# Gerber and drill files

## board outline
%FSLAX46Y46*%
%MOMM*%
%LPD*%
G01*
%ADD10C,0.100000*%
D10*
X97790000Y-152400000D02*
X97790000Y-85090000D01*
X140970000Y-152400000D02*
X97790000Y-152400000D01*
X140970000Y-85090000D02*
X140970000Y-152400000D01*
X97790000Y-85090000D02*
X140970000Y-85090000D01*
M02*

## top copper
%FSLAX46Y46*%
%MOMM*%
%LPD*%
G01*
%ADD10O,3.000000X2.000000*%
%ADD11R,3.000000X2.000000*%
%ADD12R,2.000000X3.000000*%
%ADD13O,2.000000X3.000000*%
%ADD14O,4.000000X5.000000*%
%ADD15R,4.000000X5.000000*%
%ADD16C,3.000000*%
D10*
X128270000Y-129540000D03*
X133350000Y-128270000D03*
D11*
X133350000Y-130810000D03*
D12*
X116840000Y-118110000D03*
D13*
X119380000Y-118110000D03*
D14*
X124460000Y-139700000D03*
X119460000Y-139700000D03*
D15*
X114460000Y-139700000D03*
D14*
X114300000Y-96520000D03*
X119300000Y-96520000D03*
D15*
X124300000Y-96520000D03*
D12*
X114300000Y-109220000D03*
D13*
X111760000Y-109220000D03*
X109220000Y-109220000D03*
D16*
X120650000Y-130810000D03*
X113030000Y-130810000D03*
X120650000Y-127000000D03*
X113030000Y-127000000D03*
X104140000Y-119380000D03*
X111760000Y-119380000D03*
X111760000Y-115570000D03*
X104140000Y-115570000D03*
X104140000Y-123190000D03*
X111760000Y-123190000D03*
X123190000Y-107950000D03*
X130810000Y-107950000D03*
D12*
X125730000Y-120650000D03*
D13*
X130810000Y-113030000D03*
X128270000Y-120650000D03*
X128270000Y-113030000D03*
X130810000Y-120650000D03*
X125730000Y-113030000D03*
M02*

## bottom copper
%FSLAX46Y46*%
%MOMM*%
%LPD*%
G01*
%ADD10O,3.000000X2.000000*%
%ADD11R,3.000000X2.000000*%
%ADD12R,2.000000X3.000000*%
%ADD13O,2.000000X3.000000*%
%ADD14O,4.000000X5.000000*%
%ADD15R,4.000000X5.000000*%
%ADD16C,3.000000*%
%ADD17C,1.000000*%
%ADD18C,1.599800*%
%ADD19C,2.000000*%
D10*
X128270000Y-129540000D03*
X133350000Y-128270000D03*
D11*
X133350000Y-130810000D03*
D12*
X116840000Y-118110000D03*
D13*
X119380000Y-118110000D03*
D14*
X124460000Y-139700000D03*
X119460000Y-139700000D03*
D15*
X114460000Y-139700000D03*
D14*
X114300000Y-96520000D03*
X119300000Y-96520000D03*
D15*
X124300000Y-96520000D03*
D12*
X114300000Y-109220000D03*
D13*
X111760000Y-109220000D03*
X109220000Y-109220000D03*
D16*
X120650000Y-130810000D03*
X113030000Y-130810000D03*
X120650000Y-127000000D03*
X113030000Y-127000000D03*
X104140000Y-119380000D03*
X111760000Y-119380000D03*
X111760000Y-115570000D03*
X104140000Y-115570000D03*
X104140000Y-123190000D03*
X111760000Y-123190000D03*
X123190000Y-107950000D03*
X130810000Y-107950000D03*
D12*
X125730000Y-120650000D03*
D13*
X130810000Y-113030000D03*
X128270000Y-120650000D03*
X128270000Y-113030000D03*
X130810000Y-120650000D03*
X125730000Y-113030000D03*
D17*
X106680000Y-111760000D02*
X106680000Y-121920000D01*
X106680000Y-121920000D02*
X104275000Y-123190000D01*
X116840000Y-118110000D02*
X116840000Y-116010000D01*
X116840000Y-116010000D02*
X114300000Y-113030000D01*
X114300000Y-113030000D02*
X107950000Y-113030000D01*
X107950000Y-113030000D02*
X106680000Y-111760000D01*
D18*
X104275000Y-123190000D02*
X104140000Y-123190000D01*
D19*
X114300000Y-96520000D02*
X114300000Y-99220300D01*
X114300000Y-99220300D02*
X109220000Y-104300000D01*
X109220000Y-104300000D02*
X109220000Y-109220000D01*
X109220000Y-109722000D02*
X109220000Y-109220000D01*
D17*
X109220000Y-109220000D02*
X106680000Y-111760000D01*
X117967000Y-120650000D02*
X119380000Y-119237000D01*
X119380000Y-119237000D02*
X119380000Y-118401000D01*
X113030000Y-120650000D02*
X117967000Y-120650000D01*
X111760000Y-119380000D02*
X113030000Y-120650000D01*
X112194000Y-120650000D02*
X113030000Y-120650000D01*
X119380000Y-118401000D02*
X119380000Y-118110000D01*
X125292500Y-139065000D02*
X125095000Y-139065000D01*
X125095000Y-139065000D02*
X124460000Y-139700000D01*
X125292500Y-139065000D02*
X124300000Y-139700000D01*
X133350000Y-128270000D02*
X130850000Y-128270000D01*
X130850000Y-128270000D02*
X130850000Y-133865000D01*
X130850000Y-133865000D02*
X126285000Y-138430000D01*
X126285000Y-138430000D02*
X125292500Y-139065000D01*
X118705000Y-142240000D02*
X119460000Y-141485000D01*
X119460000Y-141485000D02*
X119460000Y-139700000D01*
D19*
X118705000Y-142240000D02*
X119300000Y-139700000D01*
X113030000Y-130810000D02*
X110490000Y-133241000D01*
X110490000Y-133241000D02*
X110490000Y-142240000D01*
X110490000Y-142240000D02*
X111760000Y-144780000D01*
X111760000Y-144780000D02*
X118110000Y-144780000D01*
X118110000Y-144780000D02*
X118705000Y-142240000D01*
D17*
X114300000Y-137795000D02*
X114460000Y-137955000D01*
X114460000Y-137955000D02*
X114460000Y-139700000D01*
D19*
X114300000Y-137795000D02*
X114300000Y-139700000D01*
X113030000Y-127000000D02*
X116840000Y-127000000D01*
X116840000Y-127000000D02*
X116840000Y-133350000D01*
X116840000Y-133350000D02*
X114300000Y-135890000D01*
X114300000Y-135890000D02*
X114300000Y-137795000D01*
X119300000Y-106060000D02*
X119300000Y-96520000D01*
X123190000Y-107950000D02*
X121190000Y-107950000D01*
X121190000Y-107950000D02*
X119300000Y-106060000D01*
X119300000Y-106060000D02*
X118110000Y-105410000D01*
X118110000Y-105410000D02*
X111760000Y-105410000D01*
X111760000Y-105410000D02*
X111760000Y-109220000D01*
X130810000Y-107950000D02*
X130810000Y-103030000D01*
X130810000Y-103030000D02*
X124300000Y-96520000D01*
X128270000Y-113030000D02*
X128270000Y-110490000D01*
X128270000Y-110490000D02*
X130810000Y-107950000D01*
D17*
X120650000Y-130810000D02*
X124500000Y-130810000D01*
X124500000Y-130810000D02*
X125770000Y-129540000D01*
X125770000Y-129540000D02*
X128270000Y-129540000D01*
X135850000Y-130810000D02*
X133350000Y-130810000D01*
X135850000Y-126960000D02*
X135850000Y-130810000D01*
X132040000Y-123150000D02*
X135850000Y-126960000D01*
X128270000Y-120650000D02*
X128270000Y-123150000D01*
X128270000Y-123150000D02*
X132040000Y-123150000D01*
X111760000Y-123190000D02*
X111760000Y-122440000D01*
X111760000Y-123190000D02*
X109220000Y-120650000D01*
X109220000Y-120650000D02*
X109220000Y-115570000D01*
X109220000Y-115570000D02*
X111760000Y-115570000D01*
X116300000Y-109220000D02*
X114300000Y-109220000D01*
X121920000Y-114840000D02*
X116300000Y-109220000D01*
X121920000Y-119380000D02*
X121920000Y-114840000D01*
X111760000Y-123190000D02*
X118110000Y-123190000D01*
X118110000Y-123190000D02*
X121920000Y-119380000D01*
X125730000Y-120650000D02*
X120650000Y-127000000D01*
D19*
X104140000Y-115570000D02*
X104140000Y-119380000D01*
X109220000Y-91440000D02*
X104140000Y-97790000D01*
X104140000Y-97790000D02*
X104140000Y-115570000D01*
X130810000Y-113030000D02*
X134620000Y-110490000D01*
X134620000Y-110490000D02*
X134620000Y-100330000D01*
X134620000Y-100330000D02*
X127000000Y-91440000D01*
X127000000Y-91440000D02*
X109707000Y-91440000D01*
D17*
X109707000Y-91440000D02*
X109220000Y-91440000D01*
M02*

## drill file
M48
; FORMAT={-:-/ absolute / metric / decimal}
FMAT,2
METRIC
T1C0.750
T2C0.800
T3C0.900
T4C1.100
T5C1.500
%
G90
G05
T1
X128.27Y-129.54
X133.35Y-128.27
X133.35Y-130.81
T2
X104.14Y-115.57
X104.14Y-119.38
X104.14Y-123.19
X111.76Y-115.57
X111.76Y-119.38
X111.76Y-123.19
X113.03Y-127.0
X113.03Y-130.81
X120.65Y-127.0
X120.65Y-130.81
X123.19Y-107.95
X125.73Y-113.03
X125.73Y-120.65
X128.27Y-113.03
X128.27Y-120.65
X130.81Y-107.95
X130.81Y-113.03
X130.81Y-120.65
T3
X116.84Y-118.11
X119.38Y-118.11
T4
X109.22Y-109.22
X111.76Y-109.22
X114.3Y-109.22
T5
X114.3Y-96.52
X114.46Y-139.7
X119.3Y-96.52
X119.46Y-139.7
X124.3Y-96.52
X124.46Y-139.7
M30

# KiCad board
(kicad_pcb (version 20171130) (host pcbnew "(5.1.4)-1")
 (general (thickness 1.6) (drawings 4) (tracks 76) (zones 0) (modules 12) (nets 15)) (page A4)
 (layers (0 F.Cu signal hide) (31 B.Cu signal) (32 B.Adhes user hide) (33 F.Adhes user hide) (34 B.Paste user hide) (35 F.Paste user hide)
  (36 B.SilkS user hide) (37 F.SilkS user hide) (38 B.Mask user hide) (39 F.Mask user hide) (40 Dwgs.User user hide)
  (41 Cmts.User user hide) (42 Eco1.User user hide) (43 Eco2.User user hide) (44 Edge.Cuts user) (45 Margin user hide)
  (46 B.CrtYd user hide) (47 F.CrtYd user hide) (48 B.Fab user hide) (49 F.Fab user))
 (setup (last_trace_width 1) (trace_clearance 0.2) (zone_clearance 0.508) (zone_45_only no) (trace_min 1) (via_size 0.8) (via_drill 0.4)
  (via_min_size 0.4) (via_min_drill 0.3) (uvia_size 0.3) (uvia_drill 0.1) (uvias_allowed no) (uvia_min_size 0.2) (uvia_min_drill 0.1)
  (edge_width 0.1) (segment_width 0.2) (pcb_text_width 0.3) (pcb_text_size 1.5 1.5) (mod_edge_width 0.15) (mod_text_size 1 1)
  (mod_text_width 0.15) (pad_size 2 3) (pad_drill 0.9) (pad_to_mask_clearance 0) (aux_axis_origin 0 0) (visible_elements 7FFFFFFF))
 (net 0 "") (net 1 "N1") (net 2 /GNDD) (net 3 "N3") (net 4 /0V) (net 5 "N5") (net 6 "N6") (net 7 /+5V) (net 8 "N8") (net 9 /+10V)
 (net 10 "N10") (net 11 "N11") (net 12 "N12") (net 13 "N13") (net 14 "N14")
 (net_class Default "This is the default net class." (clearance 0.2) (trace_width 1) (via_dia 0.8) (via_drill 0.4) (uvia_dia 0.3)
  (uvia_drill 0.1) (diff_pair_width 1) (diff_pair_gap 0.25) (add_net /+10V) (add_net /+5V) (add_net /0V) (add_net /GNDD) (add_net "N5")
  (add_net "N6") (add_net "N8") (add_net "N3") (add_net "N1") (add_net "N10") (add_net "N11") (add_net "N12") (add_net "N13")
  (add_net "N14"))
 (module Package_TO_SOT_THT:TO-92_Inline (layer F.Cu) (at 133.35 130.81 90)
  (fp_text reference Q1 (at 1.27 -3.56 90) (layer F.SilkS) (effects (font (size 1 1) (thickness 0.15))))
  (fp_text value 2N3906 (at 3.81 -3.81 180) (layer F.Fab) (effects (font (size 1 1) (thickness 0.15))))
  (pad 2 thru_hole oval (at 1.27 -5.08 90) (size 2 3) (drill 0.75) (layers *.Cu *.Mask) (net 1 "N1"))
  (pad 3 thru_hole oval (at 2.54 0 90) (size 2 3) (drill 0.75) (layers *.Cu *.Mask) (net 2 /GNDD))
  (pad 1 thru_hole rect (at 0 0 90) (size 2 3) (drill 0.75) (layers *.Cu *.Mask) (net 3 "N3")))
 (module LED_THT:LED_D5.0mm (layer F.Cu) (at 116.84 118.11)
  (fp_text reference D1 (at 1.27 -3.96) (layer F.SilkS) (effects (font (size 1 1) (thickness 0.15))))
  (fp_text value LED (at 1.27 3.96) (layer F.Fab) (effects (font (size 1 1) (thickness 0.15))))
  (pad 1 thru_hole rect (at 0 0) (size 2 3) (drill 0.9) (layers *.Cu *.Mask) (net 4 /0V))
  (pad 2 thru_hole oval (at 2.54 0) (size 2 3) (drill 0.9) (layers *.Cu *.Mask) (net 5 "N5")))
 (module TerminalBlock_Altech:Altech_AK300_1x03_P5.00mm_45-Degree (layer F.Cu) (at 114.46 139.7)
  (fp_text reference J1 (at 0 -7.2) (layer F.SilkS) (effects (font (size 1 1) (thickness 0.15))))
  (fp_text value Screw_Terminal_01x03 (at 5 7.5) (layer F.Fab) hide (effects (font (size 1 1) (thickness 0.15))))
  (pad 3 thru_hole oval (at 10 0) (size 4 5) (drill 1.5) (layers *.Cu *.Mask) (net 2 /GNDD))
  (pad 2 thru_hole oval (at 5 0) (size 4 5) (drill 1.5) (layers *.Cu *.Mask) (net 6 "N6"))
  (pad 1 thru_hole rect (at 0 0) (size 4 5) (drill 1.5) (layers *.Cu *.Mask) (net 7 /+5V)))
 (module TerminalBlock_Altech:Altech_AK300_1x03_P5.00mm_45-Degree (layer F.Cu) (at 114.3 96.52)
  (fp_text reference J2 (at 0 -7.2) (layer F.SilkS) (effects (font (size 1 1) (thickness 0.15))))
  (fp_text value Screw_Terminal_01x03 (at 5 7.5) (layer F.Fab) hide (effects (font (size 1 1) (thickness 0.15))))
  (pad 1 thru_hole oval (at 0 0) (size 4 5) (drill 1.5) (layers *.Cu *.Mask) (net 4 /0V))
  (pad 2 thru_hole oval (at 5 0) (size 4 5) (drill 1.5) (layers *.Cu *.Mask) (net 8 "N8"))
  (pad 3 thru_hole rect (at 10 0) (size 4 5) (drill 1.5) (layers *.Cu *.Mask) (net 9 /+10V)))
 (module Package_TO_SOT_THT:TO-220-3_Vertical (layer F.Cu) (at 114.3 109.22 180)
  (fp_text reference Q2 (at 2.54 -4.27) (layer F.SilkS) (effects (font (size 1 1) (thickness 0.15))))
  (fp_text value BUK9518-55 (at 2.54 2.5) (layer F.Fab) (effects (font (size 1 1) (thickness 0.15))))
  (pad 1 thru_hole rect (at 0 0 180) (size 2 3) (drill 1.1) (layers *.Cu *.Mask) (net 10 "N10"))
  (pad 2 thru_hole oval (at 2.54 0 180) (size 2 3) (drill 1.1) (layers *.Cu *.Mask) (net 8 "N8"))
  (pad 3 thru_hole oval (at 5.08 0 180) (size 2 3) (drill 1.1) (layers *.Cu *.Mask) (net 4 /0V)))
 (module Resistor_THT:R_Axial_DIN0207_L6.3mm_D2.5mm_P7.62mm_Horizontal (layer F.Cu) (at 120.65 130.81 180)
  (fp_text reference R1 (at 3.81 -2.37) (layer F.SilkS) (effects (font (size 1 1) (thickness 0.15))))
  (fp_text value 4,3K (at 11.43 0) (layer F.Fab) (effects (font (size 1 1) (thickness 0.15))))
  (pad 1 thru_hole circle (at 0 0 180) (size 3 3) (drill 0.8) (layers *.Cu *.Mask) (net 1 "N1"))
  (pad 2 thru_hole circle (at 7.62 0 180) (size 3 3) (drill 0.8) (layers *.Cu *.Mask) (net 6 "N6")))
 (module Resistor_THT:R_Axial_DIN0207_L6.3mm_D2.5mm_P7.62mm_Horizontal (layer F.Cu) (at 120.65 127 180)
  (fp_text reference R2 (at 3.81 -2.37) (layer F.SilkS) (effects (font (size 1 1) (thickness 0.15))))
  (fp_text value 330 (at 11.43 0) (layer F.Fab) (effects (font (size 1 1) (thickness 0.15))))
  (pad 1 thru_hole circle (at 0 0 180) (size 3 3) (drill 0.8) (layers *.Cu *.Mask) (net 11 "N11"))
  (pad 2 thru_hole circle (at 7.62 0 180) (size 3 3) (drill 0.8) (layers *.Cu *.Mask) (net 7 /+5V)))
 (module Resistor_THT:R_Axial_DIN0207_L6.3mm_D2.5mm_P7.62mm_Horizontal (layer F.Cu) (at 111.76 119.38 180)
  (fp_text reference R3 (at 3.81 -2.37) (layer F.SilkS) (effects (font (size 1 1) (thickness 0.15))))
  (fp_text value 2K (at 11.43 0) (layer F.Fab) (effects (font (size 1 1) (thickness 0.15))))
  (pad 2 thru_hole circle (at 7.62 0 180) (size 3 3) (drill 0.8) (layers *.Cu *.Mask) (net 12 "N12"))
  (pad 1 thru_hole circle (at 0 0 180) (size 3 3) (drill 0.8) (layers *.Cu *.Mask) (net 5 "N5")))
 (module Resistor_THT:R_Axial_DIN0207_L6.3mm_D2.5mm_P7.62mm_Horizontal (layer F.Cu) (at 104.14 115.57)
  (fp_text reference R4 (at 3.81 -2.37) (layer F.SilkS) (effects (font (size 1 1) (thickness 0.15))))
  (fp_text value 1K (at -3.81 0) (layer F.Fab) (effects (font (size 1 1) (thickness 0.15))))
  (pad 2 thru_hole circle (at 7.62 0) (size 3 3) (drill 0.8) (layers *.Cu *.Mask) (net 10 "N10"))
  (pad 1 thru_hole circle (at 0 0) (size 3 3) (drill 0.8) (layers *.Cu *.Mask) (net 12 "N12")))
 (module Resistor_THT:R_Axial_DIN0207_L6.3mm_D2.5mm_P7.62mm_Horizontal (layer F.Cu) (at 104.14 123.19)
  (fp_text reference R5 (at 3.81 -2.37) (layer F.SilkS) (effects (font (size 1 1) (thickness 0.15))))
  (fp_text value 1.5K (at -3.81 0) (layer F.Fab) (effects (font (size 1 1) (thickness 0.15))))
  (pad 1 thru_hole circle (at 0 0) (size 3 3) (drill 0.8) (layers *.Cu *.Mask) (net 4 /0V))
  (pad 2 thru_hole circle (at 7.62 0) (size 3 3) (drill 0.8) (layers *.Cu *.Mask) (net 10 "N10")))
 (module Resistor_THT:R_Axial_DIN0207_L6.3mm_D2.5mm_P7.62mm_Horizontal (layer F.Cu) (at 130.81 107.95 180)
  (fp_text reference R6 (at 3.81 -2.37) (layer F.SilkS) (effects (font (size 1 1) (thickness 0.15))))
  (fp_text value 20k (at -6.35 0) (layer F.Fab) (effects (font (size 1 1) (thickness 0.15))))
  (pad 2 thru_hole circle (at 7.62 0 180) (size 3 3) (drill 0.8) (layers *.Cu *.Mask) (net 8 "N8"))
  (pad 1 thru_hole circle (at 0 0 180) (size 3 3) (drill 0.8) (layers *.Cu *.Mask) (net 9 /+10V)))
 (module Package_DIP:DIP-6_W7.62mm (layer F.Cu) (at 125.73 120.65 90)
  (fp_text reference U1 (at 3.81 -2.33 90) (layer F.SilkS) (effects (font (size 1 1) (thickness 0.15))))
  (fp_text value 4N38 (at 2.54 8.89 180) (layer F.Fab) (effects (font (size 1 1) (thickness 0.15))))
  (pad 1 thru_hole rect (at 0 0 90) (size 3 2) (drill 0.8) (layers *.Cu *.Mask) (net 11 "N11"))
  (pad 4 thru_hole oval (at 7.62 5.08 90) (size 3 2) (drill 0.8) (layers *.Cu *.Mask) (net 12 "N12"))
  (pad 2 thru_hole oval (at 0 2.54 90) (size 3 2) (drill 0.8) (layers *.Cu *.Mask) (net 3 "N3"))
  (pad 5 thru_hole oval (at 7.62 2.54 90) (size 3 2) (drill 0.8) (layers *.Cu *.Mask) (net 9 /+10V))
  (pad 3 thru_hole oval (at 0 5.08 90) (size 3 2) (drill 0.8) (layers *.Cu *.Mask) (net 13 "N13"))
  (pad 6 thru_hole oval (at 7.62 0 90) (size 3 2) (drill 0.8) (layers *.Cu *.Mask) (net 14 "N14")))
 (gr_line (start 97.79 152.4) (end 97.79 85.09) (layer Edge.Cuts) (width 0.1))
 (gr_line (start 140.97 152.4) (end 97.79 152.4) (layer Edge.Cuts) (width 0.1))
 (gr_line (start 140.97 85.09) (end 140.97 152.4) (layer Edge.Cuts) (width 0.1))
 (gr_line (start 97.79 85.09) (end 140.97 85.09) (layer Edge.Cuts) (width 0.1))
 (segment (start 106.68 111.76) (end 106.68 121.92) (width 1) (layer B.Cu) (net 4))
 (segment (start 106.68 121.92) (end 104.275 123.19) (width 1) (layer B.Cu) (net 4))
 (segment (start 116.84 118.11) (end 116.84 116.01) (width 1) (layer B.Cu) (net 4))
 (segment (start 116.84 116.01) (end 114.3 113.03) (width 1) (layer B.Cu) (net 4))
 (segment (start 114.3 113.03) (end 107.95 113.03) (width 1) (layer B.Cu) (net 4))
 (segment (start 107.95 113.03) (end 106.68 111.76) (width 1) (layer B.Cu) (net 4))
 (segment (start 104.275 123.19) (end 104.14 123.19) (width 1.5998) (layer B.Cu) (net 4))
 (segment (start 114.3 96.52) (end 114.3 99.2203) (width 2) (layer B.Cu) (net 4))
 (segment (start 114.3 99.2203) (end 109.22 104.3) (width 2) (layer B.Cu) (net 4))
 (segment (start 109.22 104.3) (end 109.22 109.22) (width 2) (layer B.Cu) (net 4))
 (segment (start 109.22 109.722) (end 109.22 109.22) (width 2) (layer B.Cu) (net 4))
 (segment (start 109.22 109.22) (end 106.68 111.76) (width 1) (layer B.Cu) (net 4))
 (segment (start 117.967 120.65) (end 119.38 119.237) (width 1) (layer B.Cu) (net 5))
 (segment (start 119.38 119.237) (end 119.38 118.401) (width 1) (layer B.Cu) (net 5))
 (segment (start 113.03 120.65) (end 117.967 120.65) (width 1) (layer B.Cu) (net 5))
 (segment (start 111.76 119.38) (end 113.03 120.65) (width 1) (layer B.Cu) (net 5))
 (segment (start 112.194 120.65) (end 113.03 120.65) (width 1) (layer B.Cu) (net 5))
 (segment (start 119.38 118.401) (end 119.38 118.11) (width 1) (layer B.Cu) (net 5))
 (segment (start 125.2925 139.065) (end 125.095 139.065) (width 1) (layer B.Cu) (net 2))
 (segment (start 125.095 139.065) (end 124.46 139.7) (width 1) (layer B.Cu) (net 2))
 (segment (start 125.2925 139.065) (end 124.3 139.7) (width 1) (layer B.Cu) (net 2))
 (segment (start 133.35 128.27) (end 130.85 128.27) (width 1) (layer B.Cu) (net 2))
 (segment (start 130.85 128.27) (end 130.85 133.865) (width 1) (layer B.Cu) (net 2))
 (segment (start 130.85 133.865) (end 126.285 138.43) (width 1) (layer B.Cu) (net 2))
 (segment (start 126.285 138.43) (end 125.2925 139.065) (width 1) (layer B.Cu) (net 2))
 (segment (start 118.705 142.24) (end 119.46 141.485) (width 1) (layer B.Cu) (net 6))
 (segment (start 119.46 141.485) (end 119.46 139.7) (width 1) (layer B.Cu) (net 6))
 (segment (start 118.705 142.24) (end 119.3 139.7) (width 2) (layer B.Cu) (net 6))
 (segment (start 113.03 130.81) (end 110.49 133.241) (width 2) (layer B.Cu) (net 6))
 (segment (start 110.49 133.241) (end 110.49 142.24) (width 2) (layer B.Cu) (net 6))
 (segment (start 110.49 142.24) (end 111.76 144.78) (width 2) (layer B.Cu) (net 6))
 (segment (start 111.76 144.78) (end 118.11 144.78) (width 2) (layer B.Cu) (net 6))
 (segment (start 118.11 144.78) (end 118.705 142.24) (width 2) (layer B.Cu) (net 6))
 (segment (start 114.3 137.795) (end 114.46 137.955) (width 1) (layer B.Cu) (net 7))
 (segment (start 114.46 137.955) (end 114.46 139.7) (width 1) (layer B.Cu) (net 7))
 (segment (start 114.3 137.795) (end 114.3 139.7) (width 2) (layer B.Cu) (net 7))
 (segment (start 113.03 127) (end 116.84 127) (width 2) (layer B.Cu) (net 7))
 (segment (start 116.84 127) (end 116.84 133.35) (width 2) (layer B.Cu) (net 7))
 (segment (start 116.84 133.35) (end 114.3 135.89) (width 2) (layer B.Cu) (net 7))
 (segment (start 114.3 135.89) (end 114.3 137.795) (width 2) (layer B.Cu) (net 7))
 (segment (start 119.3 106.06) (end 119.3 96.52) (width 2) (layer B.Cu) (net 8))
 (segment (start 123.19 107.95) (end 121.19 107.95) (width 2) (layer B.Cu) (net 8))
 (segment (start 121.19 107.95) (end 119.3 106.06) (width 2) (layer B.Cu) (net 8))
 (segment (start 119.3 106.06) (end 118.11 105.41) (width 2) (layer B.Cu) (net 8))
 (segment (start 118.11 105.41) (end 111.76 105.41) (width 2) (layer B.Cu) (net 8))
 (segment (start 111.76 105.41) (end 111.76 109.22) (width 2) (layer B.Cu) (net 8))
 (segment (start 130.81 107.95) (end 130.81 103.03) (width 2) (layer B.Cu) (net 9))
 (segment (start 130.81 103.03) (end 124.3 96.52) (width 2) (layer B.Cu) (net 9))
 (segment (start 128.27 113.03) (end 128.27 110.49) (width 2) (layer B.Cu) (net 9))
 (segment (start 128.27 110.49) (end 130.81 107.95) (width 2) (layer B.Cu) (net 9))
 (segment (start 120.65 130.81) (end 124.5 130.81) (width 1) (layer B.Cu) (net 1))
 (segment (start 124.5 130.81) (end 125.77 129.54) (width 1) (layer B.Cu) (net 1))
 (segment (start 125.77 129.54) (end 128.27 129.54) (width 1) (layer B.Cu) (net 1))
 (segment (start 135.85 130.81) (end 133.35 130.81) (width 1) (layer B.Cu) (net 3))
 (segment (start 135.85 126.96) (end 135.85 130.81) (width 1) (layer B.Cu) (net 3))
 (segment (start 132.04 123.15) (end 135.85 126.96) (width 1) (layer B.Cu) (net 3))
 (segment (start 128.27 120.65) (end 128.27 123.15) (width 1) (layer B.Cu) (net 3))
 (segment (start 128.27 123.15) (end 132.04 123.15) (width 1) (layer B.Cu) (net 3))
 (segment (start 111.76 123.19) (end 111.76 122.44) (width 1) (layer B.Cu) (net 10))
 (segment (start 111.76 123.19) (end 109.22 120.65) (width 1) (layer B.Cu) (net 10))
 (segment (start 109.22 120.65) (end 109.22 115.57) (width 1) (layer B.Cu) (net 10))
 (segment (start 109.22 115.57) (end 111.76 115.57) (width 1) (layer B.Cu) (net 10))
 (segment (start 116.3 109.22) (end 114.3 109.22) (width 1) (layer B.Cu) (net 10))
 (segment (start 121.92 114.84) (end 116.3 109.22) (width 1) (layer B.Cu) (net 10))
 (segment (start 121.92 119.38) (end 121.92 114.84) (width 1) (layer B.Cu) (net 10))
 (segment (start 111.76 123.19) (end 118.11 123.19) (width 1) (layer B.Cu) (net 10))
 (segment (start 118.11 123.19) (end 121.92 119.38) (width 1) (layer B.Cu) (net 10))
 (segment (start 125.73 120.65) (end 120.65 127) (width 1) (layer B.Cu) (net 11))
 (segment (start 104.14 115.57) (end 104.14 119.38) (width 2) (layer B.Cu) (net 12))
 (segment (start 109.22 91.44) (end 104.14 97.79) (width 2) (layer B.Cu) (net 12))
 (segment (start 104.14 97.79) (end 104.14 115.57) (width 2) (layer B.Cu) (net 12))
 (segment (start 130.81 113.03) (end 134.62 110.49) (width 2) (layer B.Cu) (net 12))
 (segment (start 134.62 110.49) (end 134.62 100.33) (width 2) (layer B.Cu) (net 12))
 (segment (start 134.62 100.33) (end 127 91.44) (width 2) (layer B.Cu) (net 12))
 (segment (start 127 91.44) (end 109.707 91.44) (width 2) (layer B.Cu) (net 12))
 (segment (start 109.707 91.44) (end 109.22 91.44) (width 1) (layer B.Cu) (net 12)))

